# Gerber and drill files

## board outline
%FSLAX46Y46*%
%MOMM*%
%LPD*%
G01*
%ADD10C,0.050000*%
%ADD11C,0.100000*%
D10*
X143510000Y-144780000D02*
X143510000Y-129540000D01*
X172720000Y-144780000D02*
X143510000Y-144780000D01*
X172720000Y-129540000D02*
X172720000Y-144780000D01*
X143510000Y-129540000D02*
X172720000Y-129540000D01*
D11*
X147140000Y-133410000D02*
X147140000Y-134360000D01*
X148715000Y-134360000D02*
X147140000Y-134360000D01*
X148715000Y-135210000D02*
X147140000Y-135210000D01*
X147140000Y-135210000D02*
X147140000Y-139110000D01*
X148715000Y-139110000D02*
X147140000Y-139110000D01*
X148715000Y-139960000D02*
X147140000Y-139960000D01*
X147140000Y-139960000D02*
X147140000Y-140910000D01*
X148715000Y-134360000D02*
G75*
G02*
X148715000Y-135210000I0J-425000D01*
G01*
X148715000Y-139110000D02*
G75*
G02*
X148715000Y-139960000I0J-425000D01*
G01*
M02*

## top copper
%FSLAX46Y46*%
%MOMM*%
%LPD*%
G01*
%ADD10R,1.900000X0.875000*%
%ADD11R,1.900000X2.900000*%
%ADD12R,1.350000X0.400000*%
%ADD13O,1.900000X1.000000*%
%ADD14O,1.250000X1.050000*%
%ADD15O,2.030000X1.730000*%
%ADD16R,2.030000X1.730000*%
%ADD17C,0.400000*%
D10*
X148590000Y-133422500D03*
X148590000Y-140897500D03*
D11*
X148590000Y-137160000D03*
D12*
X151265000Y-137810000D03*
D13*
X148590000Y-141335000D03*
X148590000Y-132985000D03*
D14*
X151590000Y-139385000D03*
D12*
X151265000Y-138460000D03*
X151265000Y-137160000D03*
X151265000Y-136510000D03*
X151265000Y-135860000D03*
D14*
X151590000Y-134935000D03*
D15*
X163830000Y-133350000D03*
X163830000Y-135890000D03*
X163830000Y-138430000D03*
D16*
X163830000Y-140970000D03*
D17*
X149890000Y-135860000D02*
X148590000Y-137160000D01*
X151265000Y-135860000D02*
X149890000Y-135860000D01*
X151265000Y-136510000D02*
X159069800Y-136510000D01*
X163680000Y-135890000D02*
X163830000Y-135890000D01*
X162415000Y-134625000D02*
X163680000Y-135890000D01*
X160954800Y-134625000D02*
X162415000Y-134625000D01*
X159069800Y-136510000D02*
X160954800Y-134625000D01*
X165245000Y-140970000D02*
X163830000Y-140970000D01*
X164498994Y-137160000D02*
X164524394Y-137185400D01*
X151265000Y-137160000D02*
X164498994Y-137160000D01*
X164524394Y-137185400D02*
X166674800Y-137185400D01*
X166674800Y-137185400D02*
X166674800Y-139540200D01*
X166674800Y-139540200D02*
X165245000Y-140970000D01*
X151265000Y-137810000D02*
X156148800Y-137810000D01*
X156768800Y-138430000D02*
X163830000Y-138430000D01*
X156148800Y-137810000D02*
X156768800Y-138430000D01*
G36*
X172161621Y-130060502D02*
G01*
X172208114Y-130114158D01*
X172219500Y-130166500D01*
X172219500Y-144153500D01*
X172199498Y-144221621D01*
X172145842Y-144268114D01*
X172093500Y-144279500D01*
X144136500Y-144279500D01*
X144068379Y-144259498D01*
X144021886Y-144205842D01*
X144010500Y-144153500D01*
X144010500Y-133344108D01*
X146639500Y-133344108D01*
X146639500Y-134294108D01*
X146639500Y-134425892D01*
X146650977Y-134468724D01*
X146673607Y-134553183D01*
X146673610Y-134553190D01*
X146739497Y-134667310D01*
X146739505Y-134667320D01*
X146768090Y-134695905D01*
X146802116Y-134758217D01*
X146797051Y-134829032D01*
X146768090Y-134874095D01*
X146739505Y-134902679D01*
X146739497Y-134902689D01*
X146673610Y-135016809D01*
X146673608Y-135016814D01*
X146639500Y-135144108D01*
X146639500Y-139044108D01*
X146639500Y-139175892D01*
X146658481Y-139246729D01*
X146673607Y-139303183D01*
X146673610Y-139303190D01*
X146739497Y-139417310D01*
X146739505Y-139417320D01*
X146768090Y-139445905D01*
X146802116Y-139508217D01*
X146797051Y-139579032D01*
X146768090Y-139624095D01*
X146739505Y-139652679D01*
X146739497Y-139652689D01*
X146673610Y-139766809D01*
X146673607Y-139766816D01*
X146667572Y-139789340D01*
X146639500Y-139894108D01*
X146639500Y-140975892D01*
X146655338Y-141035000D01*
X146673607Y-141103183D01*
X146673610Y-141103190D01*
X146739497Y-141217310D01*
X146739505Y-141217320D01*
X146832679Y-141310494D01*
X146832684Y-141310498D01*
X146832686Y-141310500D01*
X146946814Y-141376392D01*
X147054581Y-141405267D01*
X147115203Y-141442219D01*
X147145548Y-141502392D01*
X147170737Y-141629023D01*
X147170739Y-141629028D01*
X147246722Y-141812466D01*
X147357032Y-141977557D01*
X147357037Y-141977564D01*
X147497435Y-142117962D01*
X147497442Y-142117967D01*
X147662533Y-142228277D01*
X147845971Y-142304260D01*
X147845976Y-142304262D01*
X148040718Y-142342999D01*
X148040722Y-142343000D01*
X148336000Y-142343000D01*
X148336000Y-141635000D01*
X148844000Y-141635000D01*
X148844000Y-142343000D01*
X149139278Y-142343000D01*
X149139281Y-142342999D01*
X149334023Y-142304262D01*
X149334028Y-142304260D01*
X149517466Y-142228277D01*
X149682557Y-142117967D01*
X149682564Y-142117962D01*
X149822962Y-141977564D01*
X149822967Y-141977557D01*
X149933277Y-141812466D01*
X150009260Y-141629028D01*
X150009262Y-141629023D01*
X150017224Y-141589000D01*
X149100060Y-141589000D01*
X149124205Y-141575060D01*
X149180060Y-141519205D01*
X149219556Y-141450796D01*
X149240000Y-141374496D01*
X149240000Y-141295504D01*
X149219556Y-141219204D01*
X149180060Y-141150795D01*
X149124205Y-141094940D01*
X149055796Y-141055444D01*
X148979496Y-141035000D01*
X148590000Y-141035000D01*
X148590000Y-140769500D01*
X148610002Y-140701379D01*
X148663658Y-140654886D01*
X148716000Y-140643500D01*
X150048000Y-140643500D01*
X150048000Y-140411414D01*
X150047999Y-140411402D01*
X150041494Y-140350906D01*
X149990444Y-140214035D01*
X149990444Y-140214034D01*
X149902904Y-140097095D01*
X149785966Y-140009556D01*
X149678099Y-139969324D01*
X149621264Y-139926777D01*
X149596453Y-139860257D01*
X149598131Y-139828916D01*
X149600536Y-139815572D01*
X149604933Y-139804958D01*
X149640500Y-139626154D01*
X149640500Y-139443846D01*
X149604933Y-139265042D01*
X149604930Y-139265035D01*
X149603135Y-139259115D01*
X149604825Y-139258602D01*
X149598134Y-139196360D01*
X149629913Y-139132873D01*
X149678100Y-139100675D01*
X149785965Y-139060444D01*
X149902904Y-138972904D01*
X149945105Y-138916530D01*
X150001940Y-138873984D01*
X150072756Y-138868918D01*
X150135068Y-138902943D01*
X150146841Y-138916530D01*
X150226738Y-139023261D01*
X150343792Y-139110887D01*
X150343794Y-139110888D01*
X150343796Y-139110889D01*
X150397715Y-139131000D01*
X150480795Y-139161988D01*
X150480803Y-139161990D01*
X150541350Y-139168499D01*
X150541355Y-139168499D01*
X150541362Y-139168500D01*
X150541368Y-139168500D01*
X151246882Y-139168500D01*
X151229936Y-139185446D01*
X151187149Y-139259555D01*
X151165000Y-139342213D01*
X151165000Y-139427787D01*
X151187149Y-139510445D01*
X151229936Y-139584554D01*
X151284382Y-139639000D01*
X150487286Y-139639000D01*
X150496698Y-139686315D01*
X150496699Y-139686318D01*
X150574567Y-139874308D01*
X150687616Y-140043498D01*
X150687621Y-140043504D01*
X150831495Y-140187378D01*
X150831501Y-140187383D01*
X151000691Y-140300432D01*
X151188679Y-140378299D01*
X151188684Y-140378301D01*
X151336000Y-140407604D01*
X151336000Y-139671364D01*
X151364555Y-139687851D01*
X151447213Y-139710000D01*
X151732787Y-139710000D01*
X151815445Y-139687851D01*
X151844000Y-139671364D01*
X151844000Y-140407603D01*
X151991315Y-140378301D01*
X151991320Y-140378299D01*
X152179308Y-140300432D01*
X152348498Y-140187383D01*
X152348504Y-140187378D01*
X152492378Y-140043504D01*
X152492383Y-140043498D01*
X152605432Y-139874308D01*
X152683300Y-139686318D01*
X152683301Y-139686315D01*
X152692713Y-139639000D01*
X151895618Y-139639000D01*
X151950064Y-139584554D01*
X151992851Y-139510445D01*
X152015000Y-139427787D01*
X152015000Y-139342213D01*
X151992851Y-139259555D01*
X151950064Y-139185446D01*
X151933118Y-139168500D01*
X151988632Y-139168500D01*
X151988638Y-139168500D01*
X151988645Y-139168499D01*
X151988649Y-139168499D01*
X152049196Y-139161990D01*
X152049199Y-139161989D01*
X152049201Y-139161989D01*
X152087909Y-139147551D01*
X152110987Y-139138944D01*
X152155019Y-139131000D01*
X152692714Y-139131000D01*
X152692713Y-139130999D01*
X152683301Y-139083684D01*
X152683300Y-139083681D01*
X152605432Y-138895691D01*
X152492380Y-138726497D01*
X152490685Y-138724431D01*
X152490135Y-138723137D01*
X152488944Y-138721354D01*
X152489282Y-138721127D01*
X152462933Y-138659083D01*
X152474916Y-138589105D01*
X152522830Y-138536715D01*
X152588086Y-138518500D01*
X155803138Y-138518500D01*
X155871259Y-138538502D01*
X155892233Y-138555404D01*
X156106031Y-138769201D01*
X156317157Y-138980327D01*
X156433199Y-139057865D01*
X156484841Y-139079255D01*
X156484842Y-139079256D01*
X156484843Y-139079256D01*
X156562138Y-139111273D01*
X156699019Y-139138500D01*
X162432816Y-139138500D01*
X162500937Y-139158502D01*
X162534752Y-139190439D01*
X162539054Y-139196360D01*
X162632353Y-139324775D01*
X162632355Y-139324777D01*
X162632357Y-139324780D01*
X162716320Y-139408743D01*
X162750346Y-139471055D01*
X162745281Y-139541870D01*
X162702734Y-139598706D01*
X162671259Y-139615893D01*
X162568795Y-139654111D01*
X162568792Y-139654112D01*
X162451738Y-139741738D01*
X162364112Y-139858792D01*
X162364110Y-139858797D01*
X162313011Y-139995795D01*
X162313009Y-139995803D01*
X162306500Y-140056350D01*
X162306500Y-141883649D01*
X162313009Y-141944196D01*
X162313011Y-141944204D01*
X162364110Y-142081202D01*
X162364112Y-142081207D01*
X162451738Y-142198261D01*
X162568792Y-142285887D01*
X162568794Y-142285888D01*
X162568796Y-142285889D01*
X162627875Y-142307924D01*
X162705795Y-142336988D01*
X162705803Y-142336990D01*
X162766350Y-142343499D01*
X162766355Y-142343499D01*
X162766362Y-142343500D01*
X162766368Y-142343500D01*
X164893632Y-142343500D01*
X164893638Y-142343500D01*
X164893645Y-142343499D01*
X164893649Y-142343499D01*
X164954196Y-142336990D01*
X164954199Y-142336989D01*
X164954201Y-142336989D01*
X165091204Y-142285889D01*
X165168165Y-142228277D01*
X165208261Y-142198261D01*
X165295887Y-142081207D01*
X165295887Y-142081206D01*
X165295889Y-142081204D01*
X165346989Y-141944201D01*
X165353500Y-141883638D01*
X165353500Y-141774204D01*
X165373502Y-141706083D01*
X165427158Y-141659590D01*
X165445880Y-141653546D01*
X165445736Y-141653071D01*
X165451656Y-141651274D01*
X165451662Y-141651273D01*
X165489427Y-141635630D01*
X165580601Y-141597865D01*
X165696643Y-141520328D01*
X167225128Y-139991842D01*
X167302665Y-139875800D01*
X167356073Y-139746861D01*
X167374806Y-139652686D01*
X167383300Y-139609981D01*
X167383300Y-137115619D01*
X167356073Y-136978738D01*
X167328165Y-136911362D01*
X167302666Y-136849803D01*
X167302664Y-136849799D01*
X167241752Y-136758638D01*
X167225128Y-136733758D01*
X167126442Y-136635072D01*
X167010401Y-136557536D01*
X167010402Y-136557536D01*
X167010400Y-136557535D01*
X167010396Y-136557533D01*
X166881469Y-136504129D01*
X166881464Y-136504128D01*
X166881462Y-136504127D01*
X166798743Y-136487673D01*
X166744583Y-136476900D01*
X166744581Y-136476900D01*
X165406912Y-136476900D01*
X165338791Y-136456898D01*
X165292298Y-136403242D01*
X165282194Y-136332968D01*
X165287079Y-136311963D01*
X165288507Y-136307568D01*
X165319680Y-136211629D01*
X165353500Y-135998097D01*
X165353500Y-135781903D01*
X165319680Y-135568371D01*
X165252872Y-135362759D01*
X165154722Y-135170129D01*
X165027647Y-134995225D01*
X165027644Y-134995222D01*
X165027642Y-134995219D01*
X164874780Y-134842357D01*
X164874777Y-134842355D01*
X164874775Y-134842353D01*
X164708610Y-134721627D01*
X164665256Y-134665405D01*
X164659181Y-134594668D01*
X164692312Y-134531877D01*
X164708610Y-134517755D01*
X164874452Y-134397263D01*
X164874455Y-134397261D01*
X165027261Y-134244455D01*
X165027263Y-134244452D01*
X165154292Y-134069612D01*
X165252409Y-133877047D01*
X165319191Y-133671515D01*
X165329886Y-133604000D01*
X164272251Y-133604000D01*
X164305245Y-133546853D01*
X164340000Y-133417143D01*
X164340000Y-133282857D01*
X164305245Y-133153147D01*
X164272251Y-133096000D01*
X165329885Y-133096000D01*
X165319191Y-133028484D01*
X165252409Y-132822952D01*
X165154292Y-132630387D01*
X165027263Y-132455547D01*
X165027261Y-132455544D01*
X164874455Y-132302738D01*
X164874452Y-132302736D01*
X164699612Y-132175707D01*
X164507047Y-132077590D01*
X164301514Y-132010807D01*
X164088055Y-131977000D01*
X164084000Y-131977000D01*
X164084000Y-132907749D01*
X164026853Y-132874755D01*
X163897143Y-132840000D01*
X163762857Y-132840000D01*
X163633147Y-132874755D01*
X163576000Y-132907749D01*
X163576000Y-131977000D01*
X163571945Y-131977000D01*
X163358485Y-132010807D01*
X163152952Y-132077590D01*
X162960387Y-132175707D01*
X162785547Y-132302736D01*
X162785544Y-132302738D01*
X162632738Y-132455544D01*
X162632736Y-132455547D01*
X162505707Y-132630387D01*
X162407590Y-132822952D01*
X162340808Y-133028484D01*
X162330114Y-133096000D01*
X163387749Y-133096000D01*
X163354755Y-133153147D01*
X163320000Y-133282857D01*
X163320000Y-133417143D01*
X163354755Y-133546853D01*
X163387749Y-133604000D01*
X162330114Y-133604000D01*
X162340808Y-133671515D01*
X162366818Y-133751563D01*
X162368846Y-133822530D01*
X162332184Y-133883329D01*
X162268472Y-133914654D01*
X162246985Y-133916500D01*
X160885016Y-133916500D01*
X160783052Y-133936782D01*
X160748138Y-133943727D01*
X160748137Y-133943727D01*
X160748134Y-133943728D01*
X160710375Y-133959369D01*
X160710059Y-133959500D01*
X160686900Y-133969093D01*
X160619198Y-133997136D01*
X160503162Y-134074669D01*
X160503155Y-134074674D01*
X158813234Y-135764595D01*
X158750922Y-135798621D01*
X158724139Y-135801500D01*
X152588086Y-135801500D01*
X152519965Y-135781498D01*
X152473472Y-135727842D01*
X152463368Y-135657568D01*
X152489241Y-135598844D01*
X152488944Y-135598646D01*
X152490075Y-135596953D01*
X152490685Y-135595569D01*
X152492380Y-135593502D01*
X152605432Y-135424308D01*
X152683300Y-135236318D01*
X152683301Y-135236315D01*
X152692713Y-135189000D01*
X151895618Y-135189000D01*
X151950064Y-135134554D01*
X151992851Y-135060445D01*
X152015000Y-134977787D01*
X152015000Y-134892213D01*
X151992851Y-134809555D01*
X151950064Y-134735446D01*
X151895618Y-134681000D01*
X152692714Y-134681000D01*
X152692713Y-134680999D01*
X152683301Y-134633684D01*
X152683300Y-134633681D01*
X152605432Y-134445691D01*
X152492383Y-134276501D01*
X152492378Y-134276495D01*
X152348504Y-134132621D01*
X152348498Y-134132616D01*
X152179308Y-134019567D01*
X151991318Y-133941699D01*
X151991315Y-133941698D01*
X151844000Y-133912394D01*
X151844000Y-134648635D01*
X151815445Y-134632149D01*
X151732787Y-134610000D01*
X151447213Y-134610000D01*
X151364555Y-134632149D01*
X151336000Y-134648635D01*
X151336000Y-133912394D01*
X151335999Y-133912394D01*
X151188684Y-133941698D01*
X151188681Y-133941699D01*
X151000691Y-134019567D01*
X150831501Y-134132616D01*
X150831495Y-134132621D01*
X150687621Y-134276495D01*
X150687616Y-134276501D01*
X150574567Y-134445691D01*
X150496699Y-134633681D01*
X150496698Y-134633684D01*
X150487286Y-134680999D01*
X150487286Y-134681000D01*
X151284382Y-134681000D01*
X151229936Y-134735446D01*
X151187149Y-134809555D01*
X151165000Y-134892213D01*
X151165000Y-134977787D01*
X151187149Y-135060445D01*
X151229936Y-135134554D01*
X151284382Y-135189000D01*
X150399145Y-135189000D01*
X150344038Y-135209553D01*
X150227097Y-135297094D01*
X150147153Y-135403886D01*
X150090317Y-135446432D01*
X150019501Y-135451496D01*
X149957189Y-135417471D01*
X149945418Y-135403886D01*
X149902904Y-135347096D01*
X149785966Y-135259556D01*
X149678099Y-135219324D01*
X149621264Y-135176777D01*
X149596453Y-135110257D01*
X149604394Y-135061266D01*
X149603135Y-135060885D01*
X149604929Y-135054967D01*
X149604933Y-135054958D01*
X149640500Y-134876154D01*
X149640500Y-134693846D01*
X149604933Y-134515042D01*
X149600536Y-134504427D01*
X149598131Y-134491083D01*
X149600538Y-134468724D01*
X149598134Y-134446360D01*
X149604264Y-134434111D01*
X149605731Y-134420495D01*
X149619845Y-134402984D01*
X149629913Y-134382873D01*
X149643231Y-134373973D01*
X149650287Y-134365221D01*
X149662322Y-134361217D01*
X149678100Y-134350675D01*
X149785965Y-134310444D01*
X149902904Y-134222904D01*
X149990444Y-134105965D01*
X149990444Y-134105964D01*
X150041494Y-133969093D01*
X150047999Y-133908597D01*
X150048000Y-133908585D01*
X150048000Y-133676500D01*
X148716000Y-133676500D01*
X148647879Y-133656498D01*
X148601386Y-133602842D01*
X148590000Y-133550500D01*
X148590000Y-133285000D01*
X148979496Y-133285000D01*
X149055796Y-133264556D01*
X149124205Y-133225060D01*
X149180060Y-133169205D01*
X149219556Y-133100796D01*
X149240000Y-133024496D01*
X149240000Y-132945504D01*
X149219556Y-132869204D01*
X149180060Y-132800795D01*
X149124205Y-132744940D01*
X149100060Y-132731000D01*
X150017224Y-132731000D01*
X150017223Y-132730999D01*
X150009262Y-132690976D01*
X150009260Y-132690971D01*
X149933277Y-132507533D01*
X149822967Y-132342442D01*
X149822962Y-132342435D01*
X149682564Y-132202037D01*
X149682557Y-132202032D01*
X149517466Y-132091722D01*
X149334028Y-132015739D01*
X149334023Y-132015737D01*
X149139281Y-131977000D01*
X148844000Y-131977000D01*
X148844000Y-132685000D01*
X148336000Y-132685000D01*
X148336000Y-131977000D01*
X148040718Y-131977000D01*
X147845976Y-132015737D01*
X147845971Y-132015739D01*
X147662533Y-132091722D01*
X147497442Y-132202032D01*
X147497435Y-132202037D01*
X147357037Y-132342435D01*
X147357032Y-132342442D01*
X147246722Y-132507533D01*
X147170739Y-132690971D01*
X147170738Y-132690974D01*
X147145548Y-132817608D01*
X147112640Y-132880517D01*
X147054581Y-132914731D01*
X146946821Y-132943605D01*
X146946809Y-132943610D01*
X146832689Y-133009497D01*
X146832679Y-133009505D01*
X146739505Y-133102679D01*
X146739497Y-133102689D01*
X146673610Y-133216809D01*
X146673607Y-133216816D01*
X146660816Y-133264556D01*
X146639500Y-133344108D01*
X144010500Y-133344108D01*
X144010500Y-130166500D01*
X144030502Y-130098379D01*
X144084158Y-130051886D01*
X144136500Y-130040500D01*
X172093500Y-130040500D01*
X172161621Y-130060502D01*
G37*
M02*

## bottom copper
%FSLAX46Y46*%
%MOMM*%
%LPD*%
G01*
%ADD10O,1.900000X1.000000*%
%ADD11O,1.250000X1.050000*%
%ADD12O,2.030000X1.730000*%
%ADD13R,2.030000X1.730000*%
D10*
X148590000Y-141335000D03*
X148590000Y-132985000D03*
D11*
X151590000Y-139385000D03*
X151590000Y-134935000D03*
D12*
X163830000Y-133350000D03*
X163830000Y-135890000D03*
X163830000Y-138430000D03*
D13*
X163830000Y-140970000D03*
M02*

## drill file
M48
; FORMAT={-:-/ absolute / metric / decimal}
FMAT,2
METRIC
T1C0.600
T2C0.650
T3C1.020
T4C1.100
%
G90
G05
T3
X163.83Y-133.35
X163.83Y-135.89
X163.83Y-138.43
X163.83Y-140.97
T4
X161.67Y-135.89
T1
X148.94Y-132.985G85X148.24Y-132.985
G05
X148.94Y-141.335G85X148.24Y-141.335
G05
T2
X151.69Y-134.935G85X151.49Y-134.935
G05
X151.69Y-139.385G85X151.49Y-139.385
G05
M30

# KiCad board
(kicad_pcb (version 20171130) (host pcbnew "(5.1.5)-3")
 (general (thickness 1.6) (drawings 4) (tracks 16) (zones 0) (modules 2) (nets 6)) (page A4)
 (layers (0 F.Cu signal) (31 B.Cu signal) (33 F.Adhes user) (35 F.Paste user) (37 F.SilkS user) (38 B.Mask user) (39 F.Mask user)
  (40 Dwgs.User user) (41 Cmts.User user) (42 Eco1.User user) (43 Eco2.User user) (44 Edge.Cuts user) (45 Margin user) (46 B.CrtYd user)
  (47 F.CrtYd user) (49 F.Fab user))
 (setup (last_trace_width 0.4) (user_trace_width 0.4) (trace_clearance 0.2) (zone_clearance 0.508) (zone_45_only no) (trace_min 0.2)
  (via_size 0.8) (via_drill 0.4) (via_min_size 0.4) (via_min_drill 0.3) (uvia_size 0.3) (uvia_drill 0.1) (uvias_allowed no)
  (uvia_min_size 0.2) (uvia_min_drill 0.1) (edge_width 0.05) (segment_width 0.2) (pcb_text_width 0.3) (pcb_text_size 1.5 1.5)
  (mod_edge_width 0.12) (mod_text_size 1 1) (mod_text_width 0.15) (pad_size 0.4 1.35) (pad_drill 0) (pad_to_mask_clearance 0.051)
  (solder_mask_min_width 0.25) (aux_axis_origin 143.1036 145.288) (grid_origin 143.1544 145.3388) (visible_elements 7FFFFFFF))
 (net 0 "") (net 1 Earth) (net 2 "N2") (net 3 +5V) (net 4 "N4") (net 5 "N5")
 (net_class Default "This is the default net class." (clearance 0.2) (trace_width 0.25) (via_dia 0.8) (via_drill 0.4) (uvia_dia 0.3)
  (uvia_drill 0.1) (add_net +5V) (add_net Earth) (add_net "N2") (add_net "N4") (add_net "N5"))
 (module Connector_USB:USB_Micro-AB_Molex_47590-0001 (layer F.Cu) (at 148.59 137.16 270)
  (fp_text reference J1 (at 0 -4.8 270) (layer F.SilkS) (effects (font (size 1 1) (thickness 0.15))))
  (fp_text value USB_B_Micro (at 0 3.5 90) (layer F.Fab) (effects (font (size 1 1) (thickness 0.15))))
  (fp_line (start -3.75 1.45) (end -2.8 1.45) (layer Edge.Cuts) (width 0.1))
  (fp_line (start -2.8 -0.125) (end -2.8 1.45) (layer Edge.Cuts) (width 0.1))
  (fp_line (start -1.95 -0.125) (end -1.95 1.45) (layer Edge.Cuts) (width 0.1))
  (fp_line (start -1.95 1.45) (end 1.95 1.45) (layer Edge.Cuts) (width 0.1))
  (fp_line (start 1.95 -0.125) (end 1.95 1.45) (layer Edge.Cuts) (width 0.1))
  (fp_line (start 2.8 -0.125) (end 2.8 1.45) (layer Edge.Cuts) (width 0.1))
  (fp_line (start 2.8 1.45) (end 3.75 1.45) (layer Edge.Cuts) (width 0.1))
  (fp_arc (start -2.375 -0.125) (end -2.8 -0.125) (angle 180) (layer Edge.Cuts) (width 0.1))
  (fp_arc (start 2.375 -0.125) (end 1.95 -0.125) (angle 180) (layer Edge.Cuts) (width 0.1))
  (pad "" smd rect (at -3.5 0 270) (size 0.3 0.85) (layers F.Paste))
  (pad "" smd rect (at 3.5 0 270) (size 0.3 0.85) (layers F.Paste))
  (pad 6 smd rect (at -3.7375 0 270) (size 0.875 1.9) (layers F.Cu F.Mask) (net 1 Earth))
  (pad 6 smd rect (at 3.7375 0 270) (size 0.875 1.9) (layers F.Cu F.Mask) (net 1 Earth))
  (pad 6 smd rect (at 0 0 270) (size 2.9 1.9) (layers F.Cu F.Paste F.Mask) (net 1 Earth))
  (pad 2 smd rect (at 0.65 -2.675 270) (size 0.4 1.35) (layers F.Cu F.Paste F.Mask) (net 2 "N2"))
  (pad 6 thru_hole oval (at 4.175 0 270) (size 1 1.9) (drill oval 0.6 1.3) (layers *.Cu *.Mask) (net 1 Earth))
  (pad 6 thru_hole oval (at -4.175 0 270) (size 1 1.9) (drill oval 0.6 1.3) (layers *.Cu *.Mask) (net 1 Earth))
  (pad 6 thru_hole oval (at 2.225 -3 270) (size 1.05 1.25) (drill oval 0.65 0.85) (layers *.Cu *.Mask) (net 1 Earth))
  (pad 1 smd rect (at 1.3 -2.675 270) (size 0.4 1.35) (layers F.Cu F.Paste F.Mask) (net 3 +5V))
  (pad 3 smd rect (at 0 -2.675 270) (size 0.4 1.35) (layers F.Cu F.Paste F.Mask) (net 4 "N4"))
  (pad 4 smd rect (at -0.65 -2.675 270) (size 0.4 1.35) (layers F.Cu F.Paste F.Mask) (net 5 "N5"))
  (pad 5 smd rect (at -1.3 -2.675 270) (size 0.4 1.35) (layers F.Cu F.Paste F.Mask) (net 1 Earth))
  (pad 6 thru_hole oval (at -2.225 -3 270) (size 1.05 1.25) (drill oval 0.65 0.85) (layers *.Cu *.Mask) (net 1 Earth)))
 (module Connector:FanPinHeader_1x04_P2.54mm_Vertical (layer F.Cu) (at 163.83 140.97 90)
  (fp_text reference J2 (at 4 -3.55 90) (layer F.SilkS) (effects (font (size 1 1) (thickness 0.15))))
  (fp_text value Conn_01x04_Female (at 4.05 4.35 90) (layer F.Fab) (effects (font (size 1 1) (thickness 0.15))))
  (pad "" np_thru_hole circle (at 5.08 -2.16 180) (size 1.1 1.1) (drill 1.1) (layers *.Cu *.Mask))
  (pad 4 thru_hole oval (at 7.62 0 180) (size 2.03 1.73) (drill 1.02) (layers *.Cu *.Mask) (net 1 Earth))
  (pad 3 thru_hole oval (at 5.08 0 180) (size 2.03 1.73) (drill 1.02) (layers *.Cu *.Mask) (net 5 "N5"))
  (pad 2 thru_hole oval (at 2.54 0 180) (size 2.03 1.73) (drill 1.02) (layers *.Cu *.Mask) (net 2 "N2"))
  (pad 1 thru_hole rect (at 0 0 180) (size 2.03 1.73) (drill 1.02) (layers *.Cu *.Mask) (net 4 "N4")))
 (gr_line (start 143.51 144.78) (end 143.51 129.54) (layer Edge.Cuts) (width 0.05))
 (gr_line (start 172.72 144.78) (end 143.51 144.78) (layer Edge.Cuts) (width 0.05))
 (gr_line (start 172.72 129.54) (end 172.72 144.78) (layer Edge.Cuts) (width 0.05))
 (gr_line (start 143.51 129.54) (end 172.72 129.54) (layer Edge.Cuts) (width 0.05))
 (segment (start 149.89 135.86) (end 148.59 137.16) (width 0.4) (layer F.Cu) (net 1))
 (segment (start 151.265 135.86) (end 149.89 135.86) (width 0.4) (layer F.Cu) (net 1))
 (segment (start 151.265 136.51) (end 159.0698 136.51) (width 0.4) (layer F.Cu) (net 5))
 (segment (start 163.68 135.89) (end 163.83 135.89) (width 0.4) (layer F.Cu) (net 5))
 (segment (start 162.415 134.625) (end 163.68 135.89) (width 0.4) (layer F.Cu) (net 5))
 (segment (start 160.9548 134.625) (end 162.415 134.625) (width 0.4) (layer F.Cu) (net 5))
 (segment (start 159.0698 136.51) (end 160.9548 134.625) (width 0.4) (layer F.Cu) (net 5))
 (segment (start 165.245 140.97) (end 163.83 140.97) (width 0.4) (layer F.Cu) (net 4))
 (segment (start 164.498994 137.16) (end 164.524394 137.1854) (width 0.4) (layer F.Cu) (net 4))
 (segment (start 151.265 137.16) (end 164.498994 137.16) (width 0.4) (layer F.Cu) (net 4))
 (segment (start 164.524394 137.1854) (end 166.6748 137.1854) (width 0.4) (layer F.Cu) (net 4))
 (segment (start 166.6748 137.1854) (end 166.6748 139.5402) (width 0.4) (layer F.Cu) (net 4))
 (segment (start 166.6748 139.5402) (end 165.245 140.97) (width 0.4) (layer F.Cu) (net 4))
 (segment (start 151.265 137.81) (end 156.1488 137.81) (width 0.4) (layer F.Cu) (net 2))
 (segment (start 156.7688 138.43) (end 163.83 138.43) (width 0.4) (layer F.Cu) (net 2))
 (segment (start 156.1488 137.81) (end 156.7688 138.43) (width 0.4) (layer F.Cu) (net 2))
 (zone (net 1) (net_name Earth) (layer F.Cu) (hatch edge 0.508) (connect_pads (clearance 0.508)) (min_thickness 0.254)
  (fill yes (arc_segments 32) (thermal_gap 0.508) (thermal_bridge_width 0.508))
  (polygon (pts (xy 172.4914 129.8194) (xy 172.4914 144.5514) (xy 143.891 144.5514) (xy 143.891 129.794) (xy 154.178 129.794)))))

